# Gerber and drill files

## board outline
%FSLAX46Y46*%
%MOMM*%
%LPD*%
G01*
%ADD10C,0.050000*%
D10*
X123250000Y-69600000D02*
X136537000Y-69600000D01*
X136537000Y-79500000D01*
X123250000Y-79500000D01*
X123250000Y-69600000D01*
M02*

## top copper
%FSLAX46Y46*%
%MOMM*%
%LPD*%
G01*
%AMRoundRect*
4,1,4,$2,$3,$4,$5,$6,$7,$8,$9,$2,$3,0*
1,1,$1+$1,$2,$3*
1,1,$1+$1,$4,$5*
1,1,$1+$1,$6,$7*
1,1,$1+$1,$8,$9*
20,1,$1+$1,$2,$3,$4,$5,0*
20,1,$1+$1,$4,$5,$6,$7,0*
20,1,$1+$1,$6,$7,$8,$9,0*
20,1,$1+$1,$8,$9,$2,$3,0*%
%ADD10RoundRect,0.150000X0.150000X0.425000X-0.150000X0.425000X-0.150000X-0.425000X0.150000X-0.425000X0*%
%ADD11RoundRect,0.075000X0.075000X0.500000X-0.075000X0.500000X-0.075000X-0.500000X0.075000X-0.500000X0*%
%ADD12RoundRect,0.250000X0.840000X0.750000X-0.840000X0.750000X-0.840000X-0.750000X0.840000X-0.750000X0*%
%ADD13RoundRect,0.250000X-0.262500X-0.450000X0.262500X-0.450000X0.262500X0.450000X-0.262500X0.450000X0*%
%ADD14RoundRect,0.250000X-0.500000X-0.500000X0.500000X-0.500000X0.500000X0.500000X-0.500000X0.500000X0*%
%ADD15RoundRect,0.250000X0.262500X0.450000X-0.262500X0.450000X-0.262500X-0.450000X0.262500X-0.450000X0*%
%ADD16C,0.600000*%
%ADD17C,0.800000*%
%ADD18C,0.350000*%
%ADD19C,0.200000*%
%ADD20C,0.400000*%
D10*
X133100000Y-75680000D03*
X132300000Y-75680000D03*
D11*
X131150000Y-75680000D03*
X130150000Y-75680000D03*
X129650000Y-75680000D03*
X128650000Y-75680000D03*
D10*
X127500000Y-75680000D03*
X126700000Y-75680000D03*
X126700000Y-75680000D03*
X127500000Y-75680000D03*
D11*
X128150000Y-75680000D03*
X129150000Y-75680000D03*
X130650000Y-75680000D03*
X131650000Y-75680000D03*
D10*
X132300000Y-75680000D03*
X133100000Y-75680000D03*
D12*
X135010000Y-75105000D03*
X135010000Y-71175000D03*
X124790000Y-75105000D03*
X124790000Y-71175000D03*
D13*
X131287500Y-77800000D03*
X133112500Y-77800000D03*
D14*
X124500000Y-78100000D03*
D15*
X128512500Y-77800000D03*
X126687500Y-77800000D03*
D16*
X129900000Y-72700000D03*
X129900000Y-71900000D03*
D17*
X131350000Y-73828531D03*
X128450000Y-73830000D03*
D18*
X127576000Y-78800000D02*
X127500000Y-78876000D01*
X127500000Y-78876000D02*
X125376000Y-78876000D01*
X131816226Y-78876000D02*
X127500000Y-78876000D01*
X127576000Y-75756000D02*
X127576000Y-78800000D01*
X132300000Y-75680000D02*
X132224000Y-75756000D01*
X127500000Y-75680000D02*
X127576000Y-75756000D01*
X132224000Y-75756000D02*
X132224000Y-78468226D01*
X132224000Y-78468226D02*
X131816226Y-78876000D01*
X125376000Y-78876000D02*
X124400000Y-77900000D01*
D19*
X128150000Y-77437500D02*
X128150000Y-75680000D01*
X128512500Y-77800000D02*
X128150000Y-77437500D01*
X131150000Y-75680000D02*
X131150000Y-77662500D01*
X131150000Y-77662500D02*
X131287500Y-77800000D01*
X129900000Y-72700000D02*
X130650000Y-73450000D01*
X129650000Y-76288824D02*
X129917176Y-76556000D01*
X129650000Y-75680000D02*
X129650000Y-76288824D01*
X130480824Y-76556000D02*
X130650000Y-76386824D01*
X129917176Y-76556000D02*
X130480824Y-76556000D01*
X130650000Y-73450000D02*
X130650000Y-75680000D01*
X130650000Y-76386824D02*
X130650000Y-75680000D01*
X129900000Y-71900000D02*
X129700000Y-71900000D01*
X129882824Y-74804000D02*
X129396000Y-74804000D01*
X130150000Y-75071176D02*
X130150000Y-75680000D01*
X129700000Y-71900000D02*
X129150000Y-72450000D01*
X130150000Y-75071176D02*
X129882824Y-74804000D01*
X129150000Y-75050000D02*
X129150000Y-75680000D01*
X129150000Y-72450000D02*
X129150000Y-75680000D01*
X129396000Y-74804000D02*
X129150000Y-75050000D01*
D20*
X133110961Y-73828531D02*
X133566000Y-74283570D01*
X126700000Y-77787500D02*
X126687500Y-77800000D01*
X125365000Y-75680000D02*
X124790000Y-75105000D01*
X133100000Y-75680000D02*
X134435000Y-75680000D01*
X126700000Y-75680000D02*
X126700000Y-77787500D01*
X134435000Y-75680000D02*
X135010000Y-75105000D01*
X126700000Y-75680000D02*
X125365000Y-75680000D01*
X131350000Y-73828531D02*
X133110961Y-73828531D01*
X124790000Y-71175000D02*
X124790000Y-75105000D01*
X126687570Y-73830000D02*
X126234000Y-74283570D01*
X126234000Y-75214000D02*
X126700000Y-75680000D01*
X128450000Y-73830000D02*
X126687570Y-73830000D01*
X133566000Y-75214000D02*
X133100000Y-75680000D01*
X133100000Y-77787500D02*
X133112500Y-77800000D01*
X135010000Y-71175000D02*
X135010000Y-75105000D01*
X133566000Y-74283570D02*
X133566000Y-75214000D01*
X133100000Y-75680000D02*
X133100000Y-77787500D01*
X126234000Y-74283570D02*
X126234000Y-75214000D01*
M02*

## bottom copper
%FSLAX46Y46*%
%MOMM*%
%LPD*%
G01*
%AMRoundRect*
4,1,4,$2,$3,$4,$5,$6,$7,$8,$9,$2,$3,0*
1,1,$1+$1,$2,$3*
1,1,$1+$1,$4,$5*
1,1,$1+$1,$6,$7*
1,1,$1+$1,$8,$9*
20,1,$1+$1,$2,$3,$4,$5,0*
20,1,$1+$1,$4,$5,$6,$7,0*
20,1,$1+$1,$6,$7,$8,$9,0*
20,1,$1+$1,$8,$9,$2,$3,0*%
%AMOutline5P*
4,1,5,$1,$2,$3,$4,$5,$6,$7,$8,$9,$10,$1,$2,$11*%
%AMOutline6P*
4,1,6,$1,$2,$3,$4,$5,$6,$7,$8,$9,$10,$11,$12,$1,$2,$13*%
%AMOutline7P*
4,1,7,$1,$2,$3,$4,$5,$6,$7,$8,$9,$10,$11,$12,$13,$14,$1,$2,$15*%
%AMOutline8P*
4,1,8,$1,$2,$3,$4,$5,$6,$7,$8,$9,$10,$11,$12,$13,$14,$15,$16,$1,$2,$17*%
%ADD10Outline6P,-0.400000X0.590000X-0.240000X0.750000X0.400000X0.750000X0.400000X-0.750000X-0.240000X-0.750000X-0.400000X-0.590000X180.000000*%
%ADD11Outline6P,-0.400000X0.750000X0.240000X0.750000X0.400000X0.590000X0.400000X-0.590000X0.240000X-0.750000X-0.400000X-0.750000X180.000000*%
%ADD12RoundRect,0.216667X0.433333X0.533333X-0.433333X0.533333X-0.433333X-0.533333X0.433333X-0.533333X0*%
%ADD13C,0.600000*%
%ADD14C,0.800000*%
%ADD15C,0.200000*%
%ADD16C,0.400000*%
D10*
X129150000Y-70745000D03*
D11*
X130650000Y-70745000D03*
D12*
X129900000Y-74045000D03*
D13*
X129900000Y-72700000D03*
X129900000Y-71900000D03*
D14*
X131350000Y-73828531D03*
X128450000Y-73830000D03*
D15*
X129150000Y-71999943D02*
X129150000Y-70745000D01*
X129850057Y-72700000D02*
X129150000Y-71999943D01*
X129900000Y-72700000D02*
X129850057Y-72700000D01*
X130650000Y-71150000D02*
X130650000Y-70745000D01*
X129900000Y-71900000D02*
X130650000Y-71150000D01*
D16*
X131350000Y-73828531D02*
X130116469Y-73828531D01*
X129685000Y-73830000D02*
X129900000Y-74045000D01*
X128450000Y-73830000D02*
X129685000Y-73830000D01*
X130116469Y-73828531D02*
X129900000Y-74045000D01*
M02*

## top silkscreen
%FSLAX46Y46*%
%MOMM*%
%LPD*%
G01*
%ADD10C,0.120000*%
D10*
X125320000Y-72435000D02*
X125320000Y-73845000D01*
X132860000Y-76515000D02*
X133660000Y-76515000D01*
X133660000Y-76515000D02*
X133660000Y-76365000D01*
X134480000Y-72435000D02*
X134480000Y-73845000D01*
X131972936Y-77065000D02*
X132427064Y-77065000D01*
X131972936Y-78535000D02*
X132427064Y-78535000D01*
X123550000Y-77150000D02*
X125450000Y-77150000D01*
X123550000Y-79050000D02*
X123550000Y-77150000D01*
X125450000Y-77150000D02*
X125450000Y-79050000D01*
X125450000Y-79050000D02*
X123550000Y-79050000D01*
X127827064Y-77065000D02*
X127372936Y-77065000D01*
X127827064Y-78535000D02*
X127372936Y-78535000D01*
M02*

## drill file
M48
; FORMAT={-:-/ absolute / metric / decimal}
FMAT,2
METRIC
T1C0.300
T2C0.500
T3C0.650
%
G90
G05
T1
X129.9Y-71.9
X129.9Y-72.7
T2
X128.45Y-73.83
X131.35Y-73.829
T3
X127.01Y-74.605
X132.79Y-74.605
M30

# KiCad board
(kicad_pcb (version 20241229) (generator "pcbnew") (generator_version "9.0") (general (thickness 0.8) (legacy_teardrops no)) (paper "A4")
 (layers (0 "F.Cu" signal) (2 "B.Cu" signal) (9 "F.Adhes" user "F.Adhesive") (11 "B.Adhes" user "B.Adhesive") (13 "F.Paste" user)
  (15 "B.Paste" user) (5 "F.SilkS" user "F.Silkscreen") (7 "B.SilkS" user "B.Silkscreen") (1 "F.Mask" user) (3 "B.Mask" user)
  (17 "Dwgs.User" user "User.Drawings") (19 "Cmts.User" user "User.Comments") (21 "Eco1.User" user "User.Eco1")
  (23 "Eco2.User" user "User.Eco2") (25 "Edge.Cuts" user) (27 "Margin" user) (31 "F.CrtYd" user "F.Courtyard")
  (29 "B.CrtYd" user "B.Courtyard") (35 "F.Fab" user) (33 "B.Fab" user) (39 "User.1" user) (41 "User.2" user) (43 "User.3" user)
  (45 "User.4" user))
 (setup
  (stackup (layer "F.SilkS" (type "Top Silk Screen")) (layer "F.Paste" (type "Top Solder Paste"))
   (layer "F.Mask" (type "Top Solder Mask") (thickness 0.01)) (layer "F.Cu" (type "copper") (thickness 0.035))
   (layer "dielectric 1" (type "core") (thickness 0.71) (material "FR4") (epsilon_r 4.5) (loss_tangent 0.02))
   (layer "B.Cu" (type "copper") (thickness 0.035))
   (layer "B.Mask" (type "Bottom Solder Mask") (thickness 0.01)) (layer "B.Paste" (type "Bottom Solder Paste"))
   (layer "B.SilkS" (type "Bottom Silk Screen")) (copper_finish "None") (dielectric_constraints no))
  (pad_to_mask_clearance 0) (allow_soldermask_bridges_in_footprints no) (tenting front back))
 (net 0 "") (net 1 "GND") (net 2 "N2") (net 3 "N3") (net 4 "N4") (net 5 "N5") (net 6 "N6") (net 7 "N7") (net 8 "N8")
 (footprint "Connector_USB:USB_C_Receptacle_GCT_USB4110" (layer "F.Cu") (at 129.9 72 180)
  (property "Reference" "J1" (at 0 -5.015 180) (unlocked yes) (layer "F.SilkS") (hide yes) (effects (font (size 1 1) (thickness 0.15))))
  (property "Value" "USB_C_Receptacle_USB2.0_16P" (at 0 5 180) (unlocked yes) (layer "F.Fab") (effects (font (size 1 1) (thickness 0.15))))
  (fp_line (start 4.58 -0.435) (end 4.58 -1.845) (stroke (width 0.12) (type default)) (layer "F.SilkS"))
  (fp_line (start -2.96 -4.515) (end -3.76 -4.515) (stroke (width 0.12) (type default)) (layer "F.SilkS"))
  (fp_line (start -3.76 -4.515) (end -3.76 -4.365) (stroke (width 0.12) (type default)) (layer "F.SilkS"))
  (fp_line (start -4.58 -0.435) (end -4.58 -1.845) (stroke (width 0.12) (type default)) (layer "F.SilkS"))
  (pad "" np_thru_hole circle (at -2.89 -2.605 180) (size 0.65 0.65) (drill 0.65) (layers "*.Cu" "*.Mask"))
  (pad "" np_thru_hole circle (at 2.89 -2.605 180) (size 0.65 0.65) (drill 0.65) (layers "*.Cu" "*.Mask"))
  (pad "A1" smd roundrect (at -3.2 -3.68 180) (size 0.6 1.15) (layers "F.Cu" "F.Mask" "F.Paste") (roundrect_rratio 0.25) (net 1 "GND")
   (thermal_bridge_angle 45))
  (pad "A4" smd roundrect (at -2.4 -3.68 180) (size 0.6 1.15) (layers "F.Cu" "F.Mask" "F.Paste") (roundrect_rratio 0.25) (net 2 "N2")
   (thermal_bridge_angle 45))
  (pad "A5" smd roundrect (at -1.25 -3.68 180) (size 0.3 1.15) (layers "F.Cu" "F.Mask" "F.Paste") (roundrect_rratio 0.25) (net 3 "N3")
   (thermal_bridge_angle 45))
  (pad "A6" smd roundrect (at -0.25 -3.68 180) (size 0.3 1.15) (layers "F.Cu" "F.Mask" "F.Paste") (roundrect_rratio 0.25) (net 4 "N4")
   (thermal_bridge_angle 45))
  (pad "A7" smd roundrect (at 0.25 -3.68 180) (size 0.3 1.15) (layers "F.Cu" "F.Mask" "F.Paste") (roundrect_rratio 0.25) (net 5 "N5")
   (thermal_bridge_angle 45))
  (pad "A8" smd roundrect (at 1.25 -3.68 180) (size 0.3 1.15) (layers "F.Cu" "F.Mask" "F.Paste") (roundrect_rratio 0.25) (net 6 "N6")
   (thermal_bridge_angle 45))
  (pad "A9" smd roundrect (at 2.4 -3.68 180) (size 0.6 1.15) (layers "F.Cu" "F.Mask" "F.Paste") (roundrect_rratio 0.25) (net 2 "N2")
   (thermal_bridge_angle 45))
  (pad "A12" smd roundrect (at 3.2 -3.68 180) (size 0.6 1.15) (layers "F.Cu" "F.Mask" "F.Paste") (roundrect_rratio 0.25) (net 1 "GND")
   (thermal_bridge_angle 45))
  (pad "B1" smd roundrect (at 3.2 -3.68 180) (size 0.6 1.15) (layers "F.Cu" "F.Mask" "F.Paste") (roundrect_rratio 0.25) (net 1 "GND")
   (thermal_bridge_angle 45))
  (pad "B4" smd roundrect (at 2.4 -3.68 180) (size 0.6 1.15) (layers "F.Cu" "F.Mask" "F.Paste") (roundrect_rratio 0.25) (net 2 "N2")
   (thermal_bridge_angle 45))
  (pad "B5" smd roundrect (at 1.75 -3.68 180) (size 0.3 1.15) (layers "F.Cu" "F.Mask" "F.Paste") (roundrect_rratio 0.25) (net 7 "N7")
   (thermal_bridge_angle 45))
  (pad "B6" smd roundrect (at 0.75 -3.68 180) (size 0.3 1.15) (layers "F.Cu" "F.Mask" "F.Paste") (roundrect_rratio 0.25) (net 4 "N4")
   (thermal_bridge_angle 45))
  (pad "B7" smd roundrect (at -0.75 -3.68 180) (size 0.3 1.15) (layers "F.Cu" "F.Mask" "F.Paste") (roundrect_rratio 0.25) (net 5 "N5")
   (thermal_bridge_angle 45))
  (pad "B8" smd roundrect (at -1.75 -3.68 180) (size 0.3 1.15) (layers "F.Cu" "F.Mask" "F.Paste") (roundrect_rratio 0.25) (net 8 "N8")
   (thermal_bridge_angle 45))
  (pad "B9" smd roundrect (at -2.4 -3.68 180) (size 0.6 1.15) (layers "F.Cu" "F.Mask" "F.Paste") (roundrect_rratio 0.25) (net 2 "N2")
   (thermal_bridge_angle 45))
  (pad "B12" smd roundrect (at -3.2 -3.68 180) (size 0.6 1.15) (layers "F.Cu" "F.Mask" "F.Paste") (roundrect_rratio 0.25) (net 1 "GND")
   (thermal_bridge_angle 45))
  (pad "S1" smd roundrect (at -5.11 -3.105 180) (size 2.18 2) (layers "F.Cu" "F.Mask" "F.Paste") (roundrect_rratio 0.125) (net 1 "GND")
   (thermal_bridge_angle 45))
  (pad "S1" smd roundrect (at -5.11 0.825 180) (size 2.18 2) (layers "F.Cu" "F.Mask" "F.Paste") (roundrect_rratio 0.125) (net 1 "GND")
   (thermal_bridge_angle 45))
  (pad "S1" smd roundrect (at 5.11 -3.105 180) (size 2.18 2) (layers "F.Cu" "F.Mask" "F.Paste") (roundrect_rratio 0.125) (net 1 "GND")
   (thermal_bridge_angle 45))
  (pad "S1" smd roundrect (at 5.11 0.825 180) (size 2.18 2) (layers "F.Cu" "F.Mask" "F.Paste") (roundrect_rratio 0.125) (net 1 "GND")
   (thermal_bridge_angle 45)))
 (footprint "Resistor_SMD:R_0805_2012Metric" (layer "F.Cu") (at 132.2 77.8)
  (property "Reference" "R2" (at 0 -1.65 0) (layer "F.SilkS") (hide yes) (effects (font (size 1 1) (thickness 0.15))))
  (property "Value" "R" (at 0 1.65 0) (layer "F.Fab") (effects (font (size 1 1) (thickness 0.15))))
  (fp_line (start -0.227064 -0.735) (end 0.227064 -0.735) (stroke (width 0.12) (type solid)) (layer "F.SilkS"))
  (fp_line (start -0.227064 0.735) (end 0.227064 0.735) (stroke (width 0.12) (type solid)) (layer "F.SilkS"))
  (pad "1" smd roundrect (at -0.9125 0) (size 1.025 1.4) (layers "F.Cu" "F.Mask" "F.Paste") (roundrect_rratio 0.243902) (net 3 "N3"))
  (pad "2" smd roundrect (at 0.9125 0) (size 1.025 1.4) (layers "F.Cu" "F.Mask" "F.Paste") (roundrect_rratio 0.243902) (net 1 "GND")))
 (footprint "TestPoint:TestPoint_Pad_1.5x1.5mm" (layer "F.Cu") (at 124.5 78.1)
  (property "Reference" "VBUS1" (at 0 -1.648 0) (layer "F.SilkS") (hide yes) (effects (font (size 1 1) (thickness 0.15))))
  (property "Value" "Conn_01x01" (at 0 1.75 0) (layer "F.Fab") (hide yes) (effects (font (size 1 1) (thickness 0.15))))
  (fp_line (start -0.95 -0.95) (end 0.95 -0.95) (stroke (width 0.12) (type solid)) (layer "F.SilkS"))
  (fp_line (start -0.95 0.95) (end -0.95 -0.95) (stroke (width 0.12) (type solid)) (layer "F.SilkS"))
  (fp_line (start 0.95 -0.95) (end 0.95 0.95) (stroke (width 0.12) (type solid)) (layer "F.SilkS"))
  (fp_line (start 0.95 0.95) (end -0.95 0.95) (stroke (width 0.12) (type solid)) (layer "F.SilkS"))
  (pad "1" smd roundrect (at 0 0) (size 1.5 1.5) (layers "F.Cu" "F.Mask") (roundrect_rratio 0.1666666667) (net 2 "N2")))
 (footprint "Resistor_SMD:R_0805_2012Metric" (layer "F.Cu") (at 127.6 77.8 180)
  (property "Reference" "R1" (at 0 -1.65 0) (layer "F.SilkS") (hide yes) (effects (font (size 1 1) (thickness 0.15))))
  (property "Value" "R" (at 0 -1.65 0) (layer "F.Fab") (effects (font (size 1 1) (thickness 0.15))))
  (fp_line (start -0.227064 0.735) (end 0.227064 0.735) (stroke (width 0.12) (type solid)) (layer "F.SilkS"))
  (fp_line (start -0.227064 -0.735) (end 0.227064 -0.735) (stroke (width 0.12) (type solid)) (layer "F.SilkS"))
  (pad "1" smd roundrect (at -0.9125 0 180) (size 1.025 1.4) (layers "F.Cu" "F.Mask" "F.Paste") (roundrect_rratio 0.243902) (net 7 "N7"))
  (pad "2" smd roundrect (at 0.9125 0 180) (size 1.025 1.4) (layers "F.Cu" "F.Mask" "F.Paste") (roundrect_rratio 0.243902) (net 1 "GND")))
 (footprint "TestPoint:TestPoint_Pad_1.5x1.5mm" (layer "B.Cu") (at 128.9 70.745 180)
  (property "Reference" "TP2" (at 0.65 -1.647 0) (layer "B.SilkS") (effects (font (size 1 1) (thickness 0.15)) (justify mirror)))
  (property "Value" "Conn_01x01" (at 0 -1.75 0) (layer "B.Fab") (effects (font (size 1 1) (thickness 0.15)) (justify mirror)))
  (pad "1" smd roundrect (at -0.25 0 180) (size 0.8 1.5) (layers "B.Cu" "B.Mask") (roundrect_rratio 0) (chamfer_ratio 0.2)
   (chamfer top_left bottom_left) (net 5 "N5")))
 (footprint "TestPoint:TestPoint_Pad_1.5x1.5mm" (layer "B.Cu") (at 130.9 70.745 180)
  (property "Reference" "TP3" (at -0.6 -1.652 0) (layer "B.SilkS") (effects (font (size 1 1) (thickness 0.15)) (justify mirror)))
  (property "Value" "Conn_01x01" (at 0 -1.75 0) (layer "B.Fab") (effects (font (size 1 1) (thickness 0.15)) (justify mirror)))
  (pad "1" smd roundrect (at 0.25 0 180) (size 0.8 1.5) (layers "B.Cu" "B.Mask") (roundrect_rratio 0) (chamfer_ratio 0.2)
   (chamfer top_right bottom_right) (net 4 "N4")))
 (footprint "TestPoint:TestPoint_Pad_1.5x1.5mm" (layer "B.Cu") (at 129.9 74.045 180)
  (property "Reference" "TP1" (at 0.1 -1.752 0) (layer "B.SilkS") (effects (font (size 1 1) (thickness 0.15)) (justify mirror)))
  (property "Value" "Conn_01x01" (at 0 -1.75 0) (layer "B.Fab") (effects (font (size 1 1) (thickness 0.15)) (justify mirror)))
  (pad "1" smd roundrect (at 0 0 180) (size 1.3 1.5) (layers "B.Cu" "B.Mask") (roundrect_rratio 0.1666666667) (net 1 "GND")))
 (gr_rect (start 123.25 69.6) (end 136.537 79.5) (stroke (width 0.05) (type default)) (fill no) (layer "Edge.Cuts"))
 (segment (start 127.576 78.8) (end 127.5 78.876) (width 0.35) (layer "F.Cu") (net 2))
 (segment (start 127.5 78.876) (end 125.376 78.876) (width 0.35) (layer "F.Cu") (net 2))
 (segment (start 131.816226 78.876) (end 127.5 78.876) (width 0.35) (layer "F.Cu") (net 2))
 (segment (start 127.576 75.756) (end 127.576 78.8) (width 0.35) (layer "F.Cu") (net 2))
 (segment (start 132.3 75.68) (end 132.224 75.756) (width 0.35) (layer "F.Cu") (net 2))
 (segment (start 127.5 75.68) (end 127.576 75.756) (width 0.35) (layer "F.Cu") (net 2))
 (segment (start 132.224 75.756) (end 132.224 78.468226) (width 0.35) (layer "F.Cu") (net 2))
 (segment (start 132.224 78.468226) (end 131.816226 78.876) (width 0.35) (layer "F.Cu") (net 2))
 (segment (start 125.376 78.876) (end 124.4 77.9) (width 0.35) (layer "F.Cu") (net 2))
 (segment (start 128.15 77.4375) (end 128.15 75.68) (width 0.2) (layer "F.Cu") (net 7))
 (segment (start 128.5125 77.8) (end 128.15 77.4375) (width 0.2) (layer "F.Cu") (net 7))
 (segment (start 131.15 75.68) (end 131.15 77.6625) (width 0.2) (layer "F.Cu") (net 3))
 (segment (start 131.15 77.6625) (end 131.2875 77.8) (width 0.2) (layer "F.Cu") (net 3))
 (segment (start 129.9 72.7) (end 130.65 73.45) (width 0.2) (layer "F.Cu") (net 5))
 (segment (start 129.65 76.288824) (end 129.917176 76.556) (width 0.2) (layer "F.Cu") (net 5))
 (segment (start 129.65 75.68) (end 129.65 76.288824) (width 0.2) (layer "F.Cu") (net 5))
 (segment (start 130.480824 76.556) (end 130.65 76.386824) (width 0.2) (layer "F.Cu") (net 5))
 (segment (start 129.917176 76.556) (end 130.480824 76.556) (width 0.2) (layer "F.Cu") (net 5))
 (segment (start 130.65 73.45) (end 130.65 75.68) (width 0.2) (layer "F.Cu") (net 5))
 (segment (start 130.65 76.386824) (end 130.65 75.68) (width 0.2) (layer "F.Cu") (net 5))
 (via (at 129.9 72.7) (size 0.6) (drill 0.3) (layers "F.Cu" "B.Cu") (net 5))
 (segment (start 129.15 71.999943) (end 129.15 70.745) (width 0.2) (layer "B.Cu") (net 5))
 (segment (start 129.850057 72.7) (end 129.15 71.999943) (width 0.2) (layer "B.Cu") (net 5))
 (segment (start 129.9 72.7) (end 129.850057 72.7) (width 0.2) (layer "B.Cu") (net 5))
 (segment (start 129.9 71.9) (end 129.7 71.9) (width 0.2) (layer "F.Cu") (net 4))
 (segment (start 129.882824 74.804) (end 129.396 74.804) (width 0.2) (layer "F.Cu") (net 4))
 (segment (start 130.15 75.071176) (end 130.15 75.68) (width 0.2) (layer "F.Cu") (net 4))
 (segment (start 129.7 71.9) (end 129.15 72.45) (width 0.2) (layer "F.Cu") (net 4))
 (segment (start 130.15 75.071176) (end 129.882824 74.804) (width 0.2) (layer "F.Cu") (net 4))
 (segment (start 129.15 75.05) (end 129.15 75.68) (width 0.2) (layer "F.Cu") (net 4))
 (segment (start 129.15 72.45) (end 129.15 75.68) (width 0.2) (layer "F.Cu") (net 4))
 (segment (start 129.396 74.804) (end 129.15 75.05) (width 0.2) (layer "F.Cu") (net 4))
 (via (at 129.9 71.9) (size 0.6) (drill 0.3) (layers "F.Cu" "B.Cu") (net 4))
 (segment (start 130.65 71.15) (end 130.65 70.745) (width 0.2) (layer "B.Cu") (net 4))
 (segment (start 129.9 71.9) (end 130.65 71.15) (width 0.2) (layer "B.Cu") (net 4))
 (segment (start 133.110961 73.828531) (end 133.566 74.28357) (width 0.4) (layer "F.Cu") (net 1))
 (segment (start 126.7 77.7875) (end 126.6875 77.8) (width 0.4) (layer "F.Cu") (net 1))
 (segment (start 125.365 75.68) (end 124.79 75.105) (width 0.4) (layer "F.Cu") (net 1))
 (segment (start 133.1 75.68) (end 134.435 75.68) (width 0.4) (layer "F.Cu") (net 1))
 (segment (start 126.7 75.68) (end 126.7 77.7875) (width 0.4) (layer "F.Cu") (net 1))
 (segment (start 134.435 75.68) (end 135.01 75.105) (width 0.4) (layer "F.Cu") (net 1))
 (segment (start 126.7 75.68) (end 125.365 75.68) (width 0.4) (layer "F.Cu") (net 1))
 (segment (start 131.35 73.828531) (end 133.110961 73.828531) (width 0.4) (layer "F.Cu") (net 1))
 (segment (start 124.79 71.175) (end 124.79 75.105) (width 0.4) (layer "F.Cu") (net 1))
 (segment (start 126.68757 73.83) (end 126.234 74.28357) (width 0.4) (layer "F.Cu") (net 1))
 (segment (start 126.234 75.214) (end 126.7 75.68) (width 0.4) (layer "F.Cu") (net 1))
 (segment (start 128.45 73.83) (end 126.68757 73.83) (width 0.4) (layer "F.Cu") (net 1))
 (segment (start 133.566 75.214) (end 133.1 75.68) (width 0.4) (layer "F.Cu") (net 1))
 (segment (start 133.1 77.7875) (end 133.1125 77.8) (width 0.4) (layer "F.Cu") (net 1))
 (segment (start 135.01 71.175) (end 135.01 75.105) (width 0.4) (layer "F.Cu") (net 1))
 (segment (start 133.566 74.28357) (end 133.566 75.214) (width 0.4) (layer "F.Cu") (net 1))
 (segment (start 133.1 75.68) (end 133.1 77.7875) (width 0.4) (layer "F.Cu") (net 1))
 (segment (start 126.234 74.28357) (end 126.234 75.214) (width 0.4) (layer "F.Cu") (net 1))
 (via (at 131.35 73.828531) (size 0.8) (drill 0.5) (layers "F.Cu" "B.Cu") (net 1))
 (via (at 128.45 73.83) (size 0.8) (drill 0.5) (layers "F.Cu" "B.Cu") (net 1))
 (segment (start 131.35 73.828531) (end 130.116469 73.828531) (width 0.4) (layer "B.Cu") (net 1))
 (segment (start 129.685 73.83) (end 129.9 74.045) (width 0.4) (layer "B.Cu") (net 1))
 (segment (start 128.45 73.83) (end 129.685 73.83) (width 0.4) (layer "B.Cu") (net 1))
 (segment (start 130.116469 73.828531) (end 129.9 74.045) (width 0.4) (layer "B.Cu") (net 1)))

